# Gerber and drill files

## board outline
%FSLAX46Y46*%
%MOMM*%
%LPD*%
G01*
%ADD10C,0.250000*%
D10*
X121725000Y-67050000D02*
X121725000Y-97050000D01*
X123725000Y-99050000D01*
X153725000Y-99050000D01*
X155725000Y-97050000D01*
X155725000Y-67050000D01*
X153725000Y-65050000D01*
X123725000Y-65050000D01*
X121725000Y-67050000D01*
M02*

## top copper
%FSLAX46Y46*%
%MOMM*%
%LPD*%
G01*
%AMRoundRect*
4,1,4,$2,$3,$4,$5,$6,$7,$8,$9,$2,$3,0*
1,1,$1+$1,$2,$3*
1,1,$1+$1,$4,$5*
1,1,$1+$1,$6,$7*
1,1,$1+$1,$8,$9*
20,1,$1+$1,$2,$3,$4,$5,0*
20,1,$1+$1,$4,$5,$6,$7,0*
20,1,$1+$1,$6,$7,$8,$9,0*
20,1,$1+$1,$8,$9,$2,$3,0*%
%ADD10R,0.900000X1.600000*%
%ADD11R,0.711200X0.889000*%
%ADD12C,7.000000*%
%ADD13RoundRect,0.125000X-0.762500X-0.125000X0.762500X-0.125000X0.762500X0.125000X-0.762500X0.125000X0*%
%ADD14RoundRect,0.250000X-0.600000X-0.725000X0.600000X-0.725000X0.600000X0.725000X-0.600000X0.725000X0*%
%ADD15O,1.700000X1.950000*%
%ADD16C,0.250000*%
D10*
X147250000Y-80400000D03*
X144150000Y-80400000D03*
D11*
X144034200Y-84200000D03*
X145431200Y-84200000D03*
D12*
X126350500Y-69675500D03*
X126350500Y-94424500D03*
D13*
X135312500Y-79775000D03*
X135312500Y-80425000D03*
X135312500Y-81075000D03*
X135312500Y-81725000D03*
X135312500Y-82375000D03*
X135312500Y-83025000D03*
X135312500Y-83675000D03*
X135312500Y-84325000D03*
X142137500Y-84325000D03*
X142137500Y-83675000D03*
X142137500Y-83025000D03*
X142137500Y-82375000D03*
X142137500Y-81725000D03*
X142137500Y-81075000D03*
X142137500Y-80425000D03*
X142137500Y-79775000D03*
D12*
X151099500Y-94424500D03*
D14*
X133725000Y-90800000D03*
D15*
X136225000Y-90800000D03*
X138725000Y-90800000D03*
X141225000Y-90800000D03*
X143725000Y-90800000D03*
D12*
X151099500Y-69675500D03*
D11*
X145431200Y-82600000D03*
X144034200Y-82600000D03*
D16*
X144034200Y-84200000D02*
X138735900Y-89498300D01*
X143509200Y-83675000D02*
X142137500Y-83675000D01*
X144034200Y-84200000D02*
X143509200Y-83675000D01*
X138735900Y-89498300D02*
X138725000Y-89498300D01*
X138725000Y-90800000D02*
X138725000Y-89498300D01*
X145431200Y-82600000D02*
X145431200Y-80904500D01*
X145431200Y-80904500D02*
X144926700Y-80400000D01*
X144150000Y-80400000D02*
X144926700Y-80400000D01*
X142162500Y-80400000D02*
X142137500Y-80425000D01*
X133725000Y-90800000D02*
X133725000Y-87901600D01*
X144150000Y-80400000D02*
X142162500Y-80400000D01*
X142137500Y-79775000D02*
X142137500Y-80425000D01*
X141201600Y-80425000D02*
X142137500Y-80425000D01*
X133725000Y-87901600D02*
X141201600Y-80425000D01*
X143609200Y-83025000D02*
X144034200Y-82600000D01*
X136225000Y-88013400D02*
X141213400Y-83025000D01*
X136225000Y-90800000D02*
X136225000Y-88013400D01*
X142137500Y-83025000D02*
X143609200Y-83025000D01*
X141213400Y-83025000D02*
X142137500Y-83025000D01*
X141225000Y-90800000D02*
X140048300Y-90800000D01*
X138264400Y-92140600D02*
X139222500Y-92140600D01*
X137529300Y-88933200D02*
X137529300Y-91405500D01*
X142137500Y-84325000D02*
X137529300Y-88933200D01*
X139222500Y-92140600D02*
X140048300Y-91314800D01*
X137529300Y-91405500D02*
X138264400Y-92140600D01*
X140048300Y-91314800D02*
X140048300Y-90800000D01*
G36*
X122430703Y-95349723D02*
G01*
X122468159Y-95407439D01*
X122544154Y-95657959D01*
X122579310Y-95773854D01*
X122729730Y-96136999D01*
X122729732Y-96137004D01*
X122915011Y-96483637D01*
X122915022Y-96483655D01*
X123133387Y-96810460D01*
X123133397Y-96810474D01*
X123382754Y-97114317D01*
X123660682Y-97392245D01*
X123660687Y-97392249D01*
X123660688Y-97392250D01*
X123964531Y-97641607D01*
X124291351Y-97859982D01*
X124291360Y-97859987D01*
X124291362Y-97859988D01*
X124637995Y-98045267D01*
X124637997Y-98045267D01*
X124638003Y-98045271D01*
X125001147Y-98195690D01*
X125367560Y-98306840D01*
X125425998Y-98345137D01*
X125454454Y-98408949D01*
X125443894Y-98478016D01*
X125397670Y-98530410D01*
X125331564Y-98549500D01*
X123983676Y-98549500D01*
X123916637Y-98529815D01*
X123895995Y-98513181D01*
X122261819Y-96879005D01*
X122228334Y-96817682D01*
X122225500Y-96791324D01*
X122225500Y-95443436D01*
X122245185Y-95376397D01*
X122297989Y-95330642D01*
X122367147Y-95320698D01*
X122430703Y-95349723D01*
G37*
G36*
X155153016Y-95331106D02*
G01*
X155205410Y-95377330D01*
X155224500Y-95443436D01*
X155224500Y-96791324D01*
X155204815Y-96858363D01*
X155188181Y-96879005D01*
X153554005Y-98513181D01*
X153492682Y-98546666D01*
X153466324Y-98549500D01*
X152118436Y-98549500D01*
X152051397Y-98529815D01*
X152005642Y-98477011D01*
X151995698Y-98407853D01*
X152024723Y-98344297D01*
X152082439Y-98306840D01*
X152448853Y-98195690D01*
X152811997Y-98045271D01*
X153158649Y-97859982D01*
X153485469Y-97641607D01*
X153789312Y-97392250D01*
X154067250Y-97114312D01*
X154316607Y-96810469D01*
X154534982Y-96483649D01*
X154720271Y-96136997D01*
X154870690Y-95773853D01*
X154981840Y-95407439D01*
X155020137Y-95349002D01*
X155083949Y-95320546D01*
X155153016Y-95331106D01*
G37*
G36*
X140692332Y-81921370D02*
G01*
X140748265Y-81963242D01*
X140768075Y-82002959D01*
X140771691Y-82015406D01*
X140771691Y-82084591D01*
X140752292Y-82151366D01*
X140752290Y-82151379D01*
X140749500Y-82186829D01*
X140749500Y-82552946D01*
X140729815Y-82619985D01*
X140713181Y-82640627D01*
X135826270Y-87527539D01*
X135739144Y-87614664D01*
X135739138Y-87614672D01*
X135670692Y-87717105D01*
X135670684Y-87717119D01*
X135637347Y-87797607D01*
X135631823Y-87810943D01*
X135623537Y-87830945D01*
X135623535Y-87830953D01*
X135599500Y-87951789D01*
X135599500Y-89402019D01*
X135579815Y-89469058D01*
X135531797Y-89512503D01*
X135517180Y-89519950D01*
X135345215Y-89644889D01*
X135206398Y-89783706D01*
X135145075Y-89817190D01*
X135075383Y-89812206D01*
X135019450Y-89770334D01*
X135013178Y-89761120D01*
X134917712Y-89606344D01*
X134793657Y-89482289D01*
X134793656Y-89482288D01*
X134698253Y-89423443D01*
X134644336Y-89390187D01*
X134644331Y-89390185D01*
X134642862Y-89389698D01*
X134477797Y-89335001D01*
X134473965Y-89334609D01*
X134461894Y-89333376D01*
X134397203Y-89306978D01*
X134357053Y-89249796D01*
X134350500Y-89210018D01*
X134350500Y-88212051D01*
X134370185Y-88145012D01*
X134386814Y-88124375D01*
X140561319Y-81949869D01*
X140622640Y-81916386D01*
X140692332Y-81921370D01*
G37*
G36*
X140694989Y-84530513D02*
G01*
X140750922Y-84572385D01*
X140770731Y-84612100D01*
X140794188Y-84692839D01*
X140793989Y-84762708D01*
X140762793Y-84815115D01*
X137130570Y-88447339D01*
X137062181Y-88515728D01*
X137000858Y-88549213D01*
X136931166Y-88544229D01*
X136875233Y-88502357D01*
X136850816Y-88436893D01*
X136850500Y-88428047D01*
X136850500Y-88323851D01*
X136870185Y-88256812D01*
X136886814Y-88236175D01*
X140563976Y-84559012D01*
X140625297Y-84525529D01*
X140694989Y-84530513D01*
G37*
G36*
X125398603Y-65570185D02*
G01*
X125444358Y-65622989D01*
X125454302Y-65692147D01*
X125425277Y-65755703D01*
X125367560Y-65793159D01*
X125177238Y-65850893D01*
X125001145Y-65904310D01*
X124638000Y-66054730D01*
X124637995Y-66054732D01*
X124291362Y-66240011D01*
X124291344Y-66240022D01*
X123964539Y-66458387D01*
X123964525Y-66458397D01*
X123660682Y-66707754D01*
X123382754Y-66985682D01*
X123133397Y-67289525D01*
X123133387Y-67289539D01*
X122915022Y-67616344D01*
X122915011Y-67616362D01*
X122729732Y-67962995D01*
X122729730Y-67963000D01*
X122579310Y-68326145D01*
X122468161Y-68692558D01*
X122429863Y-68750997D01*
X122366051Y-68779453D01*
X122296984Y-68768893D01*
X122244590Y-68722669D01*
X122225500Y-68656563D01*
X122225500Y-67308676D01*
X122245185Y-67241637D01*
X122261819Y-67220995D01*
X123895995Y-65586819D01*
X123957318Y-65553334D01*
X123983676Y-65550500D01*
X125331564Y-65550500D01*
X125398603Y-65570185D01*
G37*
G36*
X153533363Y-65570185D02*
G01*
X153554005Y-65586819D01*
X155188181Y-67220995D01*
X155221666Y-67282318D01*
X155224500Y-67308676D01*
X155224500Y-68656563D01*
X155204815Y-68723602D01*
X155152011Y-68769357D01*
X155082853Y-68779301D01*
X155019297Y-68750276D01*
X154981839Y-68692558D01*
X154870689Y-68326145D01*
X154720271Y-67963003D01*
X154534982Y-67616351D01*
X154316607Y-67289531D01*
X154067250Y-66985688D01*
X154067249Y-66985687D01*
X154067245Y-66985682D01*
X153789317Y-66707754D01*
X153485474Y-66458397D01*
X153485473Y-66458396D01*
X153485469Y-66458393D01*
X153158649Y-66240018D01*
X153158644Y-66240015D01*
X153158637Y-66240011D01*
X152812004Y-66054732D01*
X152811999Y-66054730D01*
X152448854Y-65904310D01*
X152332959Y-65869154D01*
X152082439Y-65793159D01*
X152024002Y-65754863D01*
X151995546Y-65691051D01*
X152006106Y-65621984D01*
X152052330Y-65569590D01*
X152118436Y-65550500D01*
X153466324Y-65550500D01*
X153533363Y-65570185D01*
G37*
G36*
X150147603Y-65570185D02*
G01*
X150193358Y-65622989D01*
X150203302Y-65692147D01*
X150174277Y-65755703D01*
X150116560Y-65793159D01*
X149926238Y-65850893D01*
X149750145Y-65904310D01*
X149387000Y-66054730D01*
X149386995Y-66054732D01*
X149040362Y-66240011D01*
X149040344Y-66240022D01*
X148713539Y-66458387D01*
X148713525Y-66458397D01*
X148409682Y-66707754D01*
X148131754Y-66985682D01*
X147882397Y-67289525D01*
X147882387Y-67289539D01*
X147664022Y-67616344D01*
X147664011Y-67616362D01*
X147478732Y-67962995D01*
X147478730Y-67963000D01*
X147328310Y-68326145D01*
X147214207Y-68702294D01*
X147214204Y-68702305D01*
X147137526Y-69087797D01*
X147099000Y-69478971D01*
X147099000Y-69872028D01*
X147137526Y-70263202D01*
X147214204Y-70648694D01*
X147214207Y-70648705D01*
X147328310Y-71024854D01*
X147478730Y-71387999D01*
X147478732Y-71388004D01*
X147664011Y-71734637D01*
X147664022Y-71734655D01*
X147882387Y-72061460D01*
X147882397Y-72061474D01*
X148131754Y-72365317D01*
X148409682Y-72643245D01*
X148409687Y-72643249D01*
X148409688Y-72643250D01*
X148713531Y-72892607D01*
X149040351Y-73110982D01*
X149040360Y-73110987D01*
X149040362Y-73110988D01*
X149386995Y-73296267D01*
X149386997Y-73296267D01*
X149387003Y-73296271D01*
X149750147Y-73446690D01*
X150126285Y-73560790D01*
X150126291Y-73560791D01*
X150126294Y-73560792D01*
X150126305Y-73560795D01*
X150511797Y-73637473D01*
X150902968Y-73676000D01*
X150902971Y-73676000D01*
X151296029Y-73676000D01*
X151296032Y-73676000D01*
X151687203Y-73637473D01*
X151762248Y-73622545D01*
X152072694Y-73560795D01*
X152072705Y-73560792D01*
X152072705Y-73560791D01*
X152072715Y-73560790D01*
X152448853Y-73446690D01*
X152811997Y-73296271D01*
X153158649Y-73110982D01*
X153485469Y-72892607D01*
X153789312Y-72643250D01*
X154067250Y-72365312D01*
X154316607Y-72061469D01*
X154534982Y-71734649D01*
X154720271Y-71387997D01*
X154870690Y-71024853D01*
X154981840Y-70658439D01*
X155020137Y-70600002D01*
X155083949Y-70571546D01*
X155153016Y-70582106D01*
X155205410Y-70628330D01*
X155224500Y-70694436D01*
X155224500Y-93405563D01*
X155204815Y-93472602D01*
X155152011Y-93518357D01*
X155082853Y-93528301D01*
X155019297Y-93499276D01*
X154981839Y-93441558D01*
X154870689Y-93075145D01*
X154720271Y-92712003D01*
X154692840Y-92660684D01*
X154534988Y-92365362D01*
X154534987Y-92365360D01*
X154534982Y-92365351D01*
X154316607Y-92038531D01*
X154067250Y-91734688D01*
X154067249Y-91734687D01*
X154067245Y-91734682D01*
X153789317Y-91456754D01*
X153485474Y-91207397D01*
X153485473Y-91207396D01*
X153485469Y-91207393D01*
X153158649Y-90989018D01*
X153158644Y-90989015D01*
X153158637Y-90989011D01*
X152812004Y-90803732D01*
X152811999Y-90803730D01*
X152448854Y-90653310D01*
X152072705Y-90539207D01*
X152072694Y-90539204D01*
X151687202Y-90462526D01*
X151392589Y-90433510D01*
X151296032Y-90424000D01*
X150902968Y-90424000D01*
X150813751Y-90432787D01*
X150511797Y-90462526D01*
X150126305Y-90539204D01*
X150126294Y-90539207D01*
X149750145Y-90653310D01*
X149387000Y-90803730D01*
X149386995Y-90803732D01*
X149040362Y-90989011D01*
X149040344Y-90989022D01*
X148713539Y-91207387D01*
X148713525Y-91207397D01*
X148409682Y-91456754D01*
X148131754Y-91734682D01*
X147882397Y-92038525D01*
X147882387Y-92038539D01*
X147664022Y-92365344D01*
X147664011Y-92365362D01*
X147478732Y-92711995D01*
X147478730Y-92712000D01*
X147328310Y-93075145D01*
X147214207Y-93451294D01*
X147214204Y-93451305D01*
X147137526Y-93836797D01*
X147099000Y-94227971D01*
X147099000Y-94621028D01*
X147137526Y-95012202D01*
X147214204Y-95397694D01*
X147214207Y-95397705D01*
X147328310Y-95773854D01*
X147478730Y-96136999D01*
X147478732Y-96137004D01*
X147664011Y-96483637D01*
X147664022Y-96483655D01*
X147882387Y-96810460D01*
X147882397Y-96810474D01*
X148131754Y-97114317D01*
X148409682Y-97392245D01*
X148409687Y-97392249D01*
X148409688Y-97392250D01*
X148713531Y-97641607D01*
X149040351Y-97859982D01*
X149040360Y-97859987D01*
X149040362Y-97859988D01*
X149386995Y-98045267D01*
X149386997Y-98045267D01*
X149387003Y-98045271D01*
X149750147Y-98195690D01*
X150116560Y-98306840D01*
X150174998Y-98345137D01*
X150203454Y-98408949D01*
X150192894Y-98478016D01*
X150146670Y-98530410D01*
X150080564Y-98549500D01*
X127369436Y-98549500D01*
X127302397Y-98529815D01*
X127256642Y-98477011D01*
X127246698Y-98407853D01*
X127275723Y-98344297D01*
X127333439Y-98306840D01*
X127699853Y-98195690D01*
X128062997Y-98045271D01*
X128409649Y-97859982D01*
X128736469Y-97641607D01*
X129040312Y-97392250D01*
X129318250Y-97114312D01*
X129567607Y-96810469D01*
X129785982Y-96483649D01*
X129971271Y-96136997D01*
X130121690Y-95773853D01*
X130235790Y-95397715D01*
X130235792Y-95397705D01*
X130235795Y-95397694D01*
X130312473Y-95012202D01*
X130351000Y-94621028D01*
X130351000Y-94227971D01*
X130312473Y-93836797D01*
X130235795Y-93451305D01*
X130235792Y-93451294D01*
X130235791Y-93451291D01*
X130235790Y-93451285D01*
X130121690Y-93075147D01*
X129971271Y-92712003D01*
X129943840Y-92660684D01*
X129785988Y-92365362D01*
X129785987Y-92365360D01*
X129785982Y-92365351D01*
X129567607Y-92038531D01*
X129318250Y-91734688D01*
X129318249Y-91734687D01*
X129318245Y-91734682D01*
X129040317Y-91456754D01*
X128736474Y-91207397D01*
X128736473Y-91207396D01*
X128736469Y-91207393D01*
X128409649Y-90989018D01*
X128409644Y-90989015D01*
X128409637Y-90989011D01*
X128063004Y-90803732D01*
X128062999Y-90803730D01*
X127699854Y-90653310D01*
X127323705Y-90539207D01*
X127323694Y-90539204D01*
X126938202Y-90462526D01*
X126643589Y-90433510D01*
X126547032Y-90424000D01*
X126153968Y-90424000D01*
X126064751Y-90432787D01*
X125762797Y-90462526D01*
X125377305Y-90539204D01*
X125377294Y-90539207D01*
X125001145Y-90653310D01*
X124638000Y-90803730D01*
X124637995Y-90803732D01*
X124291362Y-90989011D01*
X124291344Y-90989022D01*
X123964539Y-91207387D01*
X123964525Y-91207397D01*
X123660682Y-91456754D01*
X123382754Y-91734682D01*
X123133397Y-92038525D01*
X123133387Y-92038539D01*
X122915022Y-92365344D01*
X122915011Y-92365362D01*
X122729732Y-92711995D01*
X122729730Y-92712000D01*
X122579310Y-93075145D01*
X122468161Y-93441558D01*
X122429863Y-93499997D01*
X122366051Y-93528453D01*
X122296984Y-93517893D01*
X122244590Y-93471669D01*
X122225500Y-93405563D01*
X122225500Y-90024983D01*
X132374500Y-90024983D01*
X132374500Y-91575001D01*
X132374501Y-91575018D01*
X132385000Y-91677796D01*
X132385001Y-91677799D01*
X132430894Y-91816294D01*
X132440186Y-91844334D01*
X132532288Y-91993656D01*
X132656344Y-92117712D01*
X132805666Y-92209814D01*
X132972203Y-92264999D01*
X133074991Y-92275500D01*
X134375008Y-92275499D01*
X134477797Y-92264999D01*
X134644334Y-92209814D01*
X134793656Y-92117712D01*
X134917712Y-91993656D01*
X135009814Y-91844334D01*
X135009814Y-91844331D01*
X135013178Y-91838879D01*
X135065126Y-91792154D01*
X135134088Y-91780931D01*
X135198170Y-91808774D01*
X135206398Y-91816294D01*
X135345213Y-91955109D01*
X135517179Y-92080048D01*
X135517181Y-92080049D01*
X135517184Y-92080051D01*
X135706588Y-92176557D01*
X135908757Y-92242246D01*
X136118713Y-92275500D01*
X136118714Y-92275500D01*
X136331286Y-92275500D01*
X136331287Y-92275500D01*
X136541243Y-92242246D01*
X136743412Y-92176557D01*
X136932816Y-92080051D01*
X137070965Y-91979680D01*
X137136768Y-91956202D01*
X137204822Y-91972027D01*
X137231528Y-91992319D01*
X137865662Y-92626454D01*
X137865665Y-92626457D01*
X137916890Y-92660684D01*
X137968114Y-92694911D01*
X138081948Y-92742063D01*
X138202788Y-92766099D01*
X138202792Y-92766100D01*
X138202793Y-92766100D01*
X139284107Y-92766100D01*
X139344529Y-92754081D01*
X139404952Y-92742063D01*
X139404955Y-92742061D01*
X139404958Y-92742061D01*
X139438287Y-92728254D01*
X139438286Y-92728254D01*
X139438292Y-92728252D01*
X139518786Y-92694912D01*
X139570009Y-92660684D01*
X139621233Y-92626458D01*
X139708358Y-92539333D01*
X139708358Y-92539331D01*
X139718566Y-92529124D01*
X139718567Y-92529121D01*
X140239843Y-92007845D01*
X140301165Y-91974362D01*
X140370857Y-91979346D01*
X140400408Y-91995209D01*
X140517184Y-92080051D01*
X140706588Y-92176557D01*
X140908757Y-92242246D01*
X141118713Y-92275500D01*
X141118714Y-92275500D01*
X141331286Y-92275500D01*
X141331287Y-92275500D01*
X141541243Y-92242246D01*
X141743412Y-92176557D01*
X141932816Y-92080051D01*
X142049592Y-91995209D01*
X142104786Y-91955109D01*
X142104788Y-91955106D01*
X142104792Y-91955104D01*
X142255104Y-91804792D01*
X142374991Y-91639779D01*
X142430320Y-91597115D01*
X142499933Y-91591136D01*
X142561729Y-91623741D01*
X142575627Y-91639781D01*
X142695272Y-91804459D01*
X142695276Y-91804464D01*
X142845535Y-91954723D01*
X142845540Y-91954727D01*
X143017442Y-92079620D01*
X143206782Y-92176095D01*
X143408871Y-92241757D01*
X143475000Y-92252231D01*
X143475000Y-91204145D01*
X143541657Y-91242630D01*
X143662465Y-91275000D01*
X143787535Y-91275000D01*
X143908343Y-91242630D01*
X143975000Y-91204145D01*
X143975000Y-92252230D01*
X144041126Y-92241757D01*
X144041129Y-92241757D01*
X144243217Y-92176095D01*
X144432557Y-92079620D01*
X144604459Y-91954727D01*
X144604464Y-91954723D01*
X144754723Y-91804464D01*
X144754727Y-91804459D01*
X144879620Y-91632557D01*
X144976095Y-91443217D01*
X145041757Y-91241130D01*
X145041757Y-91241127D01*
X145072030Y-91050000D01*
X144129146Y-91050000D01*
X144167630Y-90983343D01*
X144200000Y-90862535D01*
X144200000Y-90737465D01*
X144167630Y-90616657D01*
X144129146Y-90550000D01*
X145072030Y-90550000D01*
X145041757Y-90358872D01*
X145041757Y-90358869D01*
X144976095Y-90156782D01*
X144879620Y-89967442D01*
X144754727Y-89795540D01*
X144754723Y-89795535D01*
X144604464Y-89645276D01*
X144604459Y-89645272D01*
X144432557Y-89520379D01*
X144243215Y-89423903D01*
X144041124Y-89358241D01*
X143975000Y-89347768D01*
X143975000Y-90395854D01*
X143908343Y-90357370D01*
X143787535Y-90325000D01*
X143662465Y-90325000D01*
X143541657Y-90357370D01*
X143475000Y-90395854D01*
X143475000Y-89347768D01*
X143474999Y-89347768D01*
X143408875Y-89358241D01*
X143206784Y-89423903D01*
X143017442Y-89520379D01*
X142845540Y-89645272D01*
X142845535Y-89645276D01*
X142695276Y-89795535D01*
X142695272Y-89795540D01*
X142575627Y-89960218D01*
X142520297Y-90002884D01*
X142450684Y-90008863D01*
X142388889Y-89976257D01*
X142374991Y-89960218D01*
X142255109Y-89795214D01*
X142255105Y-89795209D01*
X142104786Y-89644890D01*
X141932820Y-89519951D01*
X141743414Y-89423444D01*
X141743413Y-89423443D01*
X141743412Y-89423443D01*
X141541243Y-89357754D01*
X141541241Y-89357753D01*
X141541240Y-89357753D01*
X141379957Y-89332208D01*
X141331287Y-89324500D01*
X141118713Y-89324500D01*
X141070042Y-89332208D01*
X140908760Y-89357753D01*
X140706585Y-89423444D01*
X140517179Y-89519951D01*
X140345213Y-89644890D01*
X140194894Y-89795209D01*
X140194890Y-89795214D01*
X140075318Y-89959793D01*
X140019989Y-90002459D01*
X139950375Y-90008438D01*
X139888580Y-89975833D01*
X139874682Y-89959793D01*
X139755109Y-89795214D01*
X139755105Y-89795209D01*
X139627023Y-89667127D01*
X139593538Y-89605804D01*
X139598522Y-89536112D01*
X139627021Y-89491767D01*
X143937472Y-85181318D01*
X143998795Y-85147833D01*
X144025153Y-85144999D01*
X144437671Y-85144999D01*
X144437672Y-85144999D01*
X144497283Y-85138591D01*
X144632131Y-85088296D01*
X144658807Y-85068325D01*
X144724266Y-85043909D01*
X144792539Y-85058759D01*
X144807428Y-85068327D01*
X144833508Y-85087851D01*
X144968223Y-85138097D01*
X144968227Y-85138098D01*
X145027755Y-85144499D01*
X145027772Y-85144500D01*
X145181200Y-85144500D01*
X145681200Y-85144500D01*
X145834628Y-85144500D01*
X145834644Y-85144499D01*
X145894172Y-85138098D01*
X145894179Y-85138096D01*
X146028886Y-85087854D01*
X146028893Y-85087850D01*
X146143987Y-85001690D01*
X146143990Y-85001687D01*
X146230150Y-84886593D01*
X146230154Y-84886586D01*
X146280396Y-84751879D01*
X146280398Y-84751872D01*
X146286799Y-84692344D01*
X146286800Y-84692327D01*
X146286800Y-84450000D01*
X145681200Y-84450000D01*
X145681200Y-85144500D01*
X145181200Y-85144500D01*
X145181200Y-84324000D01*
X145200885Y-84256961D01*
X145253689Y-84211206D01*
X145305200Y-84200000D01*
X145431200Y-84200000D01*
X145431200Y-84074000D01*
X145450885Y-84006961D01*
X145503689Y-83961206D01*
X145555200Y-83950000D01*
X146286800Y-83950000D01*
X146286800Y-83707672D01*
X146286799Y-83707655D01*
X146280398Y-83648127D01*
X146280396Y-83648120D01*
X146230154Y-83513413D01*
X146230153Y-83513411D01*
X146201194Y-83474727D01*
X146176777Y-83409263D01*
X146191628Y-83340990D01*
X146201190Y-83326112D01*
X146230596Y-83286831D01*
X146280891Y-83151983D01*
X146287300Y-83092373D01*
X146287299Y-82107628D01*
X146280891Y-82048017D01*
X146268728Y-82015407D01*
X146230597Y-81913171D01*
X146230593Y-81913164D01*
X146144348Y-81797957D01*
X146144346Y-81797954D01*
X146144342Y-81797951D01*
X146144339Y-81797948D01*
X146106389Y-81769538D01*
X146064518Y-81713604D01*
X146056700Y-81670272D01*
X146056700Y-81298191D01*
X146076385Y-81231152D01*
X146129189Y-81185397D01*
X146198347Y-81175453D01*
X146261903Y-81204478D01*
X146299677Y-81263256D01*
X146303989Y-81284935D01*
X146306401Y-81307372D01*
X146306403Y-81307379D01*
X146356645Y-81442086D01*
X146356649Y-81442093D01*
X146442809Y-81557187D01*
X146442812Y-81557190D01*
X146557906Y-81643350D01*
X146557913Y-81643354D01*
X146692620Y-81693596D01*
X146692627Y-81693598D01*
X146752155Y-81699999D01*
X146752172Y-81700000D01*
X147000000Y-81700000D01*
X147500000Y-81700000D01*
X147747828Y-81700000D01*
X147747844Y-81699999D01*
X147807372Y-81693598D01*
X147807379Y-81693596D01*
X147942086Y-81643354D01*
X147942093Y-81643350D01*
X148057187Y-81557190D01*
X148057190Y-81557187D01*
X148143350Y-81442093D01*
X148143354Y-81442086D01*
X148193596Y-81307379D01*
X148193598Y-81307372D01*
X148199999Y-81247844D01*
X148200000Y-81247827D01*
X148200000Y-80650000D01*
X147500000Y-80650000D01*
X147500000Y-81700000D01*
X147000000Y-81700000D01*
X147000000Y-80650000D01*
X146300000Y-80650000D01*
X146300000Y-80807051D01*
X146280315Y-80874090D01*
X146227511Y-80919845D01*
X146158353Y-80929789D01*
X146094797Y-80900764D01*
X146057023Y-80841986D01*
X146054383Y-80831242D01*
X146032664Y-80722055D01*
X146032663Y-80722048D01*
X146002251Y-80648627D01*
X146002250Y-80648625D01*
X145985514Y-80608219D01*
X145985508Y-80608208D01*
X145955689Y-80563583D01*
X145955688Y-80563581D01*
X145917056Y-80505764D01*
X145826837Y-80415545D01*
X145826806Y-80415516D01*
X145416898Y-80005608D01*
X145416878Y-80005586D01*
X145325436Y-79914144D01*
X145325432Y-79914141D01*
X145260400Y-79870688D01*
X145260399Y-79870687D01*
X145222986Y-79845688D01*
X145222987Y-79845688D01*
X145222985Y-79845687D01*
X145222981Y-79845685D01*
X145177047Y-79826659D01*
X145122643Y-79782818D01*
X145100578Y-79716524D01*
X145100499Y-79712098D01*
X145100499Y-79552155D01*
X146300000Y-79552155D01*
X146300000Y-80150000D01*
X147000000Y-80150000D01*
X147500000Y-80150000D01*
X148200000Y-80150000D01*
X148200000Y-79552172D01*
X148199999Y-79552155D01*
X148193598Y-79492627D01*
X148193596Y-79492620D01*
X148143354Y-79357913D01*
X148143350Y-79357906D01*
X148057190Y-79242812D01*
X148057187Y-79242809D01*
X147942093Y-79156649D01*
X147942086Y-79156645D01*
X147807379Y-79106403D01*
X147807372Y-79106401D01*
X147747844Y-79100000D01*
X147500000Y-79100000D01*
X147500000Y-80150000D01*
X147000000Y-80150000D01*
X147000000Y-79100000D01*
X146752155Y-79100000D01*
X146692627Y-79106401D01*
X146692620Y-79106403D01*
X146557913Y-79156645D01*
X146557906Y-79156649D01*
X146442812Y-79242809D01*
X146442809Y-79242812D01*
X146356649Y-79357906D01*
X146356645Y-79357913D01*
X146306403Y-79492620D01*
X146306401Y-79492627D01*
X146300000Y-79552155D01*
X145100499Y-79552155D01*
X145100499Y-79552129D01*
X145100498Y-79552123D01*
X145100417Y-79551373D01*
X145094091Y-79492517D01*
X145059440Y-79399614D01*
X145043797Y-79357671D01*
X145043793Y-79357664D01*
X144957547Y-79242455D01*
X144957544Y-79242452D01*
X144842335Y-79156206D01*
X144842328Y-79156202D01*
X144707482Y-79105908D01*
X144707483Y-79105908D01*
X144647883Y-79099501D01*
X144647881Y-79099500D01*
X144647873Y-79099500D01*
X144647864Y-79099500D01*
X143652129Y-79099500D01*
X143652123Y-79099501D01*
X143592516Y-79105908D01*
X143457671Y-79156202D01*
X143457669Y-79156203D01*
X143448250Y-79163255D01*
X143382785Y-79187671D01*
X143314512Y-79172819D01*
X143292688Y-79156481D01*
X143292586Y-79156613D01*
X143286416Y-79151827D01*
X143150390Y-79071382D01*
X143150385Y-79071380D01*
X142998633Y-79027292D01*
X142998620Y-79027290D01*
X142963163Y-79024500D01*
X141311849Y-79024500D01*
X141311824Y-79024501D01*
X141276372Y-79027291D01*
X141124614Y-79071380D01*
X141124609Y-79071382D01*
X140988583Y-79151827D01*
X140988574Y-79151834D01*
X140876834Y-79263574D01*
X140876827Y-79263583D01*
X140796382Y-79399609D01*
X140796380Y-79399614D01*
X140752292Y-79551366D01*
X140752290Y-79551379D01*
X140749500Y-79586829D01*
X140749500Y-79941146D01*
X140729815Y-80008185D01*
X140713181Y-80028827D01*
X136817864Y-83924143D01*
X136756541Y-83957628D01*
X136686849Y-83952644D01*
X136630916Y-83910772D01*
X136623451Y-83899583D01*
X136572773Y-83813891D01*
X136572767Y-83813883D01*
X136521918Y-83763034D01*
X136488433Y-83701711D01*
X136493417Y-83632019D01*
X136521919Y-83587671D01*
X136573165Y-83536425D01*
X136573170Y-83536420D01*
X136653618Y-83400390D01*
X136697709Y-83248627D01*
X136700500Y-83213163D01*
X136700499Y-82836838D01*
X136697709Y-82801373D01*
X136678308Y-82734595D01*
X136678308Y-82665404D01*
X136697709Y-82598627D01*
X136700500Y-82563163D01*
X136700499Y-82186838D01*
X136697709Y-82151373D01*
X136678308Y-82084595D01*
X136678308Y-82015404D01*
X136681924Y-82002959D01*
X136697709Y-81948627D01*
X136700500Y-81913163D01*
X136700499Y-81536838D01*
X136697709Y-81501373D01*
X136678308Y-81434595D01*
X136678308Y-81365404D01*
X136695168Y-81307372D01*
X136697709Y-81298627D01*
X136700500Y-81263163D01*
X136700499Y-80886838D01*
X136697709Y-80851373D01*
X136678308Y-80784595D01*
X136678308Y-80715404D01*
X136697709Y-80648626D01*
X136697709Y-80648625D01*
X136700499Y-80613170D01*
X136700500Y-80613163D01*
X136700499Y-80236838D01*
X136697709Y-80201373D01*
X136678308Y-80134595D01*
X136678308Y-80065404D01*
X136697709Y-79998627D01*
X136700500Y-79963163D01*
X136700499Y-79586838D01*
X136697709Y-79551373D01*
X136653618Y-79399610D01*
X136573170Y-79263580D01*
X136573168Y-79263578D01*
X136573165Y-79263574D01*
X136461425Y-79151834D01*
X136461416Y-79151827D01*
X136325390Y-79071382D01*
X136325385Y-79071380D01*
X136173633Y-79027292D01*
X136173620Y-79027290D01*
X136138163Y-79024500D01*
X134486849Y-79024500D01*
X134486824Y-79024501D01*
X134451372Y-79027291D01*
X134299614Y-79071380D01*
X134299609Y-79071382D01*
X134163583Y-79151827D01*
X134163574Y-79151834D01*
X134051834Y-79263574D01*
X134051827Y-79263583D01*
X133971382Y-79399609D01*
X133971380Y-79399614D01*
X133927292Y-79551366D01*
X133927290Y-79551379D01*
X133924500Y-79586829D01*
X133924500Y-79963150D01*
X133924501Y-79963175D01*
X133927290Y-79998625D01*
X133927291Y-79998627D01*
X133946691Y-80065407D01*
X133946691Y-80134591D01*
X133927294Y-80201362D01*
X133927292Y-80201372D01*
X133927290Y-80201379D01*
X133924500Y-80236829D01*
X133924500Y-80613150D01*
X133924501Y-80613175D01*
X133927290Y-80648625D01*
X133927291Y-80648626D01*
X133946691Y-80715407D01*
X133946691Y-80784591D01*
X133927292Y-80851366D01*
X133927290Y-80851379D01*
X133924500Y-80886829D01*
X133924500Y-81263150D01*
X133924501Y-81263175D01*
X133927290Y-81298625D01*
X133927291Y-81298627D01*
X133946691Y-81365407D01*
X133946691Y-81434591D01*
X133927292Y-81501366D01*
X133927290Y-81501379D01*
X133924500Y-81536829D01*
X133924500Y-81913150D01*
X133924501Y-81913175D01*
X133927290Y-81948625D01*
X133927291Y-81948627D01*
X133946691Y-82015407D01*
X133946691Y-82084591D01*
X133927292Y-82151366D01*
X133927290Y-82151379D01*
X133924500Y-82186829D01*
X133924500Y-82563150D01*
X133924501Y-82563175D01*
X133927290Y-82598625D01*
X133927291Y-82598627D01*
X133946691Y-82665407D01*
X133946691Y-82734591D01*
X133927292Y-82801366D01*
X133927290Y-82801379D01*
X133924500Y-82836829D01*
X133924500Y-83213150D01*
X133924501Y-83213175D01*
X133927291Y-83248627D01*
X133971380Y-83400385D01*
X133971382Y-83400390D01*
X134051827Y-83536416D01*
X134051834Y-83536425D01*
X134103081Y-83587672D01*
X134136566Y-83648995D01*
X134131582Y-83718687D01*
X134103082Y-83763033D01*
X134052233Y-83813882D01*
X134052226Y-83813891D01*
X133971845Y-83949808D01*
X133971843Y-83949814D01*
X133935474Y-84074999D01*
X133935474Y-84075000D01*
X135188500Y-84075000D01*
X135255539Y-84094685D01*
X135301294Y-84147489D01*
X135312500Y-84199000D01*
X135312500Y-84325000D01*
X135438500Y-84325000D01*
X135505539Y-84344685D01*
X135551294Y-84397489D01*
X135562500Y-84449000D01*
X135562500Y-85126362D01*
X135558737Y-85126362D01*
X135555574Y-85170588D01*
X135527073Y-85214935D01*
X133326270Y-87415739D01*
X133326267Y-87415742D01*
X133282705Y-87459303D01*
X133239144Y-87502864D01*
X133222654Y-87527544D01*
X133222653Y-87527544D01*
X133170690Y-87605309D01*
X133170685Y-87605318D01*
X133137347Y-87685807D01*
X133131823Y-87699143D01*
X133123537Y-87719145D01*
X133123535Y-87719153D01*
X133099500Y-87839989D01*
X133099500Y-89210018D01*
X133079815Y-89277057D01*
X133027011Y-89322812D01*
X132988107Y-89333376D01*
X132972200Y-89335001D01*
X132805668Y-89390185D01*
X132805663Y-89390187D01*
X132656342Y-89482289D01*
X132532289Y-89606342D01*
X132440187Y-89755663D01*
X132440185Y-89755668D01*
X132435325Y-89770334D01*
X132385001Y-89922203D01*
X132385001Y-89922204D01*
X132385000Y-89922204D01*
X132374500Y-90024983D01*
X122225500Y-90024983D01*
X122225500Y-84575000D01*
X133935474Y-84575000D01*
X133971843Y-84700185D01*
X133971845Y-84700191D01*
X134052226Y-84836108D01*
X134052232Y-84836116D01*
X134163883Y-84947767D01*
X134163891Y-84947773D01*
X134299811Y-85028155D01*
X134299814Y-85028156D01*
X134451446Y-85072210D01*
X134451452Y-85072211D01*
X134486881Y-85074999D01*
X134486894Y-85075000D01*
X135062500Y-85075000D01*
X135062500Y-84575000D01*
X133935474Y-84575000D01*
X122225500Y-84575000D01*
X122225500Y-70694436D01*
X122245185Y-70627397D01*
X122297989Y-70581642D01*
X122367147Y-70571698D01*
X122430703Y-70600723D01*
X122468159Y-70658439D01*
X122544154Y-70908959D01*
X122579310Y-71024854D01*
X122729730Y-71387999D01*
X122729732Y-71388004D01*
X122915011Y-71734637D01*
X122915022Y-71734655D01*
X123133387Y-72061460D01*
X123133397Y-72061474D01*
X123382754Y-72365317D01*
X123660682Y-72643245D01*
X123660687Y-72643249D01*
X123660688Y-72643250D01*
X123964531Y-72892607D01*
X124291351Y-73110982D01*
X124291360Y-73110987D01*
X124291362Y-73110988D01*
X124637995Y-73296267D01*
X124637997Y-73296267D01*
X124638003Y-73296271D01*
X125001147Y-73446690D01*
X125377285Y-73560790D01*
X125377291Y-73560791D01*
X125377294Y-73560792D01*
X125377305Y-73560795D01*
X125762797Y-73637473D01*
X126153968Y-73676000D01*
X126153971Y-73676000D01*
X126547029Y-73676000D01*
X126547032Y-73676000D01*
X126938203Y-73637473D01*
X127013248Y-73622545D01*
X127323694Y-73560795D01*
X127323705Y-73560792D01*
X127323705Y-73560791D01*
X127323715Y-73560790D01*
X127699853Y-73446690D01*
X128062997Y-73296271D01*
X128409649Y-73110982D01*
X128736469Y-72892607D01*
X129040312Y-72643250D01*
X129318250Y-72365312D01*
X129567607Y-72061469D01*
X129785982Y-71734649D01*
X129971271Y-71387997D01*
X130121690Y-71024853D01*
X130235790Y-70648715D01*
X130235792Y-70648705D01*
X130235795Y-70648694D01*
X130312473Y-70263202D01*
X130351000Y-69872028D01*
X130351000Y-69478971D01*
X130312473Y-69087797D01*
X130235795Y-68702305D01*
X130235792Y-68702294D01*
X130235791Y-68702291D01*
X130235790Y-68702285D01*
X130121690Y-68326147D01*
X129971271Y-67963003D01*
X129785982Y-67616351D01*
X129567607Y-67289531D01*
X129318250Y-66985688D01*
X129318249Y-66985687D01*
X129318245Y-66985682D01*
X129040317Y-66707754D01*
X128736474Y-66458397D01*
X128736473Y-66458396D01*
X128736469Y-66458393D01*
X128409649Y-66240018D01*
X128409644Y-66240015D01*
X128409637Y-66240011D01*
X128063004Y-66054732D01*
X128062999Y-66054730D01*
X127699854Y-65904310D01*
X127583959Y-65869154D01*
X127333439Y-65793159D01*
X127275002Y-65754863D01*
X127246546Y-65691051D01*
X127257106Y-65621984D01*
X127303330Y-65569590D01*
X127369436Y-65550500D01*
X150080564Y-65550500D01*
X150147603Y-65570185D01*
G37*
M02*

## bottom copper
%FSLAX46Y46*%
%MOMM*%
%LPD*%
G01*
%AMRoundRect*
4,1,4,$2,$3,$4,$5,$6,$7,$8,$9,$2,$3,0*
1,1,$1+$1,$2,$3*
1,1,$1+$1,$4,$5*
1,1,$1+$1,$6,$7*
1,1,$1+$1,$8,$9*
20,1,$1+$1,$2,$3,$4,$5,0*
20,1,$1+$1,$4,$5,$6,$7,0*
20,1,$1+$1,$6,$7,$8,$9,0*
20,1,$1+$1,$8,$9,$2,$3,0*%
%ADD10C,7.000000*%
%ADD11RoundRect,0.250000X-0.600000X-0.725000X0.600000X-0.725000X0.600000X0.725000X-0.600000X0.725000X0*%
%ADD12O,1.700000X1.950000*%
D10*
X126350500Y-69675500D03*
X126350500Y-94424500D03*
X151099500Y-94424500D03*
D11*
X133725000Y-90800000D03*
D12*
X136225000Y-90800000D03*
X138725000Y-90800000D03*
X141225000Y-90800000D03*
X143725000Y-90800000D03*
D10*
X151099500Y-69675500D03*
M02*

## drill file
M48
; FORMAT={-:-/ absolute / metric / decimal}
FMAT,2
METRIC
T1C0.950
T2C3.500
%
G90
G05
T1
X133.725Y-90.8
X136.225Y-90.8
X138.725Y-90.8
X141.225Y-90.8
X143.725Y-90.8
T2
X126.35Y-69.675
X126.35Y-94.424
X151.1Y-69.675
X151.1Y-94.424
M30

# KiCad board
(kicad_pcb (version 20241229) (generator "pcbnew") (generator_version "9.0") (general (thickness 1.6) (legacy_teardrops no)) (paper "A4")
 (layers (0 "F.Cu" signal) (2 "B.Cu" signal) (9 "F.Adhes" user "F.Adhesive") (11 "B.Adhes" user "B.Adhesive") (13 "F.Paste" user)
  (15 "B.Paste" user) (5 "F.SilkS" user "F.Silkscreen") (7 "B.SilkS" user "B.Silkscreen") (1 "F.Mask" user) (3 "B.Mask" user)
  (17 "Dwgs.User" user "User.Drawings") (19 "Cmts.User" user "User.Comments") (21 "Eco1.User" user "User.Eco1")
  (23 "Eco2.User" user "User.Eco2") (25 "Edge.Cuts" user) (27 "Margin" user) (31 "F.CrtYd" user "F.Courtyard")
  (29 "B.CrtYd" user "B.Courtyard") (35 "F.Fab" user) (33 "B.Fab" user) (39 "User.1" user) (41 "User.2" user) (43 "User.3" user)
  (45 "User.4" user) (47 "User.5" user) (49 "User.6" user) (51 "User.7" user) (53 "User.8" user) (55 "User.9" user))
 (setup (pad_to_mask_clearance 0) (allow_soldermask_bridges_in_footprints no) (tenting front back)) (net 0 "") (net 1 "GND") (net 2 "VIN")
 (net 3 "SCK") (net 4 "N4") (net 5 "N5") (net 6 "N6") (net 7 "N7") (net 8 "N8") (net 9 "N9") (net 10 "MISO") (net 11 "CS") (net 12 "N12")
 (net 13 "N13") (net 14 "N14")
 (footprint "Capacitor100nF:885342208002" (layer "F.Cu") (at 145.7 80.4 180)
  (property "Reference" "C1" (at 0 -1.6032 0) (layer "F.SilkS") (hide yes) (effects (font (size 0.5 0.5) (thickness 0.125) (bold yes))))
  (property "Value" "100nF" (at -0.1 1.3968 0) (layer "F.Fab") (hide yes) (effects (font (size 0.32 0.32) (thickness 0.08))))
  (pad "1" smd rect (at -1.55 0 180) (size 0.9 1.6) (layers "F.Cu" "F.Mask" "F.Paste") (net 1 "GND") (solder_mask_margin 0.102))
  (pad "2" smd rect (at 1.55 0 180) (size 0.9 1.6) (layers "F.Cu" "F.Mask" "F.Paste") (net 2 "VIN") (solder_mask_margin 0.102)))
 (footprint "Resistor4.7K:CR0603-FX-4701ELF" (layer "F.Cu") (at 144.7327 84.2)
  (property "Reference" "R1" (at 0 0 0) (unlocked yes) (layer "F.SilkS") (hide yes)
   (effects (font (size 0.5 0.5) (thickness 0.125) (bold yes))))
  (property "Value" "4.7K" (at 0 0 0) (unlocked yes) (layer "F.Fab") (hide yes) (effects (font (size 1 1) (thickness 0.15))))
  (pad "1" smd rect (at -0.6985 0) (size 0.7112 0.889) (layers "F.Cu" "F.Mask" "F.Paste") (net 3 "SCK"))
  (pad "2" smd rect (at 0.6985 0) (size 0.7112 0.889) (layers "F.Cu" "F.Mask" "F.Paste") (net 1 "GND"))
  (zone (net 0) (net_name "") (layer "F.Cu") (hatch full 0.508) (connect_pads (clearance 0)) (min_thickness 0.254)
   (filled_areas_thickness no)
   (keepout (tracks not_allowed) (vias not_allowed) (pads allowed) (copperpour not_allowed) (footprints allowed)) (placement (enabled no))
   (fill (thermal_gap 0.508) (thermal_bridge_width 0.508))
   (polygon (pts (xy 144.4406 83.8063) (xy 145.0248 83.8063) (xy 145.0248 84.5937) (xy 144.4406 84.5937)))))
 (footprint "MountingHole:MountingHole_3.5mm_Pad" (layer "F.Cu") (at 126.3505 69.6755)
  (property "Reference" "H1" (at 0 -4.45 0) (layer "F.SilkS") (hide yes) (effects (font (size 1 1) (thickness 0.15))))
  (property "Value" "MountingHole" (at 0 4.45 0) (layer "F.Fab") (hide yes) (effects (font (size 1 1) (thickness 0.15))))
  (pad "1" thru_hole circle (at 0 0) (size 7 7) (drill 3.5) (layers "*.Cu" "*.Mask") (remove_unused_layers no) (zone_connect 2)))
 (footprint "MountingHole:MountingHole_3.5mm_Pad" (layer "F.Cu") (at 126.3505 94.4245)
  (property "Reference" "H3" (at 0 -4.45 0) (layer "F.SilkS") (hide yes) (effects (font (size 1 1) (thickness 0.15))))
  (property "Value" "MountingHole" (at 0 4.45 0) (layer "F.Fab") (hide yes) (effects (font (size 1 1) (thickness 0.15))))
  (pad "1" thru_hole circle (at 0 0) (size 7 7) (drill 3.5) (layers "*.Cu" "*.Mask") (remove_unused_layers no) (zone_connect 2)))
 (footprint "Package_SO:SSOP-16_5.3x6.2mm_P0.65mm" (layer "F.Cu") (at 138.725 82.05)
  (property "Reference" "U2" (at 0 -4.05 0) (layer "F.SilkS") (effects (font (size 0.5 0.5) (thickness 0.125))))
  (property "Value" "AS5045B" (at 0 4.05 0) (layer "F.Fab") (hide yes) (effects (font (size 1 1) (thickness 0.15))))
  (pad "1" smd roundrect (at -3.4125 -2.275) (size 1.775 0.5) (layers "F.Cu" "F.Mask" "F.Paste") (roundrect_rratio 0.25) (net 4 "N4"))
  (pad "2" smd roundrect (at -3.4125 -1.625) (size 1.775 0.5) (layers "F.Cu" "F.Mask" "F.Paste") (roundrect_rratio 0.25) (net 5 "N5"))
  (pad "3" smd roundrect (at -3.4125 -0.975) (size 1.775 0.5) (layers "F.Cu" "F.Mask" "F.Paste") (roundrect_rratio 0.25) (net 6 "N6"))
  (pad "4" smd roundrect (at -3.4125 -0.325) (size 1.775 0.5) (layers "F.Cu" "F.Mask" "F.Paste") (roundrect_rratio 0.25) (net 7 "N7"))
  (pad "5" smd roundrect (at -3.4125 0.325) (size 1.775 0.5) (layers "F.Cu" "F.Mask" "F.Paste") (roundrect_rratio 0.25) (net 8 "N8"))
  (pad "6" smd roundrect (at -3.4125 0.975) (size 1.775 0.5) (layers "F.Cu" "F.Mask" "F.Paste") (roundrect_rratio 0.25) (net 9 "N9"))
  (pad "7" smd roundrect (at -3.4125 1.625) (size 1.775 0.5) (layers "F.Cu" "F.Mask" "F.Paste") (roundrect_rratio 0.25) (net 1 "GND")
   (zone_connect 2))
  (pad "8" smd roundrect (at -3.4125 2.275) (size 1.775 0.5) (layers "F.Cu" "F.Mask" "F.Paste") (roundrect_rratio 0.25) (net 1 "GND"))
  (pad "9" smd roundrect (at 3.4125 2.275) (size 1.775 0.5) (layers "F.Cu" "F.Mask" "F.Paste") (roundrect_rratio 0.25) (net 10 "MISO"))
  (pad "10" smd roundrect (at 3.4125 1.625) (size 1.775 0.5) (layers "F.Cu" "F.Mask" "F.Paste") (roundrect_rratio 0.25) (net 3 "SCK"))
  (pad "11" smd roundrect (at 3.4125 0.975) (size 1.775 0.5) (layers "F.Cu" "F.Mask" "F.Paste") (roundrect_rratio 0.25) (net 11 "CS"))
  (pad "12" smd roundrect (at 3.4125 0.325) (size 1.775 0.5) (layers "F.Cu" "F.Mask" "F.Paste") (roundrect_rratio 0.25) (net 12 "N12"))
  (pad "13" smd roundrect (at 3.4125 -0.325) (size 1.775 0.5) (layers "F.Cu" "F.Mask" "F.Paste") (roundrect_rratio 0.25) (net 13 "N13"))
  (pad "14" smd roundrect (at 3.4125 -0.975) (size 1.775 0.5) (layers "F.Cu" "F.Mask" "F.Paste") (roundrect_rratio 0.25) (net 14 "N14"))
  (pad "15" smd roundrect (at 3.4125 -1.625) (size 1.775 0.5) (layers "F.Cu" "F.Mask" "F.Paste") (roundrect_rratio 0.25) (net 2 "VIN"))
  (pad "16" smd roundrect (at 3.4125 -2.275) (size 1.775 0.5) (layers "F.Cu" "F.Mask" "F.Paste") (roundrect_rratio 0.25) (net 2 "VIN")))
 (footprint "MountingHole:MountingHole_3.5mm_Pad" (layer "F.Cu") (at 151.0995 94.4245)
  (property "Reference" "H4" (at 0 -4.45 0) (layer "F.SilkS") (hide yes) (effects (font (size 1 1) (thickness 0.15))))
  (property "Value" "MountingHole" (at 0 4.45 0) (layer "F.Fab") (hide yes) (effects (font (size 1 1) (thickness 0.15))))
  (pad "1" thru_hole circle (at 0 0) (size 7 7) (drill 3.5) (layers "*.Cu" "*.Mask") (remove_unused_layers no) (zone_connect 2)))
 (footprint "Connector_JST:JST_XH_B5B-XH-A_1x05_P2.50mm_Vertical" (layer "F.Cu") (at 133.725 90.8)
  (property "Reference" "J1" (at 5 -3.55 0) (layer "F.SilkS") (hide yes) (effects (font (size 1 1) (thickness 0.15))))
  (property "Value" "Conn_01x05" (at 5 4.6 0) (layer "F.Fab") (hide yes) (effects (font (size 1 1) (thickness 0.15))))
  (pad "1" thru_hole roundrect (at 0 0) (size 1.7 1.95) (drill 0.95) (layers "*.Cu" "*.Mask") (remove_unused_layers no)
   (roundrect_rratio 0.147059) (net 2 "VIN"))
  (pad "2" thru_hole oval (at 2.5 0) (size 1.7 1.95) (drill 0.95) (layers "*.Cu" "*.Mask") (remove_unused_layers no) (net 11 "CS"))
  (pad "3" thru_hole oval (at 5 0) (size 1.7 1.95) (drill 0.95) (layers "*.Cu" "*.Mask") (remove_unused_layers no) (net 3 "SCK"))
  (pad "4" thru_hole oval (at 7.5 0) (size 1.7 1.95) (drill 0.95) (layers "*.Cu" "*.Mask") (remove_unused_layers no) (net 10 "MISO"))
  (pad "5" thru_hole oval (at 10 0) (size 1.7 1.95) (drill 0.95) (layers "*.Cu" "*.Mask") (remove_unused_layers no) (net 1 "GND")))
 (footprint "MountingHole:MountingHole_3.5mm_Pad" (layer "F.Cu") (at 151.0995 69.6755)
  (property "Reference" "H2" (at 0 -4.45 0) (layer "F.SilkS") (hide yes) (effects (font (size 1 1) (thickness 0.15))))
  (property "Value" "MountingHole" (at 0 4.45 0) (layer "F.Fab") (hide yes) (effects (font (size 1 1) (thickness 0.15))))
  (pad "1" thru_hole circle (at 0 0) (size 7 7) (drill 3.5) (layers "*.Cu" "*.Mask") (remove_unused_layers no) (zone_connect 2)))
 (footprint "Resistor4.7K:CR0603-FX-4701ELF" (layer "F.Cu") (at 144.7327 82.6 180)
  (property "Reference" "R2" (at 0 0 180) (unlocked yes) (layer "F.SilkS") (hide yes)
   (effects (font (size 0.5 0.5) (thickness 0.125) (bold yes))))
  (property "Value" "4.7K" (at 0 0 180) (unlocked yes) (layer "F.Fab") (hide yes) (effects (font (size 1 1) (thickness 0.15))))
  (pad "1" smd rect (at -0.6985 0 180) (size 0.7112 0.889) (layers "F.Cu" "F.Mask" "F.Paste") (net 2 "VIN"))
  (pad "2" smd rect (at 0.6985 0 180) (size 0.7112 0.889) (layers "F.Cu" "F.Mask" "F.Paste") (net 11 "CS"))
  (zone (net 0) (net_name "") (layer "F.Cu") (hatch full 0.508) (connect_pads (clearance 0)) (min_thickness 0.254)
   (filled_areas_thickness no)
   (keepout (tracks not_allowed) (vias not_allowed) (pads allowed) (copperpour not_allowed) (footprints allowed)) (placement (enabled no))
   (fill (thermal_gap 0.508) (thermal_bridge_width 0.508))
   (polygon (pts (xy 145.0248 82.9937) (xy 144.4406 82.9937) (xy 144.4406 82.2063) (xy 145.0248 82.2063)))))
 (gr_poly
  (pts (xy 121.725 67.05) (xy 121.725 97.05) (xy 123.725 99.05) (xy 153.725 99.05) (xy 155.725 97.05) (xy 155.725 67.05) (xy 153.725 65.05)
   (xy 123.725 65.05))
  (stroke (width 0.25) (type solid)) (fill no) (layer "Edge.Cuts"))
 (segment (start 144.0342 84.2) (end 138.7359 89.4983) (width 0.25) (layer "F.Cu") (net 3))
 (segment (start 143.5092 83.675) (end 142.1375 83.675) (width 0.25) (layer "F.Cu") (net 3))
 (segment (start 144.0342 84.2) (end 143.5092 83.675) (width 0.25) (layer "F.Cu") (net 3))
 (segment (start 138.7359 89.4983) (end 138.725 89.4983) (width 0.25) (layer "F.Cu") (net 3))
 (segment (start 138.725 90.8) (end 138.725 89.4983) (width 0.25) (layer "F.Cu") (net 3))
 (segment (start 145.4312 82.6) (end 145.4312 80.9045) (width 0.25) (layer "F.Cu") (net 2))
 (segment (start 145.4312 80.9045) (end 144.9267 80.4) (width 0.25) (layer "F.Cu") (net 2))
 (segment (start 144.15 80.4) (end 144.9267 80.4) (width 0.25) (layer "F.Cu") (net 2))
 (segment (start 142.1625 80.4) (end 142.1375 80.425) (width 0.25) (layer "F.Cu") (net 2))
 (segment (start 133.725 90.8) (end 133.725 87.9016) (width 0.25) (layer "F.Cu") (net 2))
 (segment (start 144.15 80.4) (end 142.1625 80.4) (width 0.25) (layer "F.Cu") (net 2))
 (segment (start 142.1375 79.775) (end 142.1375 80.425) (width 0.25) (layer "F.Cu") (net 2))
 (segment (start 141.2016 80.425) (end 142.1375 80.425) (width 0.25) (layer "F.Cu") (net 2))
 (segment (start 133.725 87.9016) (end 141.2016 80.425) (width 0.25) (layer "F.Cu") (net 2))
 (segment (start 143.6092 83.025) (end 144.0342 82.6) (width 0.25) (layer "F.Cu") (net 11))
 (segment (start 136.225 88.0134) (end 141.2134 83.025) (width 0.25) (layer "F.Cu") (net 11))
 (segment (start 136.225 90.8) (end 136.225 88.0134) (width 0.25) (layer "F.Cu") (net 11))
 (segment (start 142.1375 83.025) (end 143.6092 83.025) (width 0.25) (layer "F.Cu") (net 11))
 (segment (start 141.2134 83.025) (end 142.1375 83.025) (width 0.25) (layer "F.Cu") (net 11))
 (segment (start 141.225 90.8) (end 140.0483 90.8) (width 0.25) (layer "F.Cu") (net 10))
 (segment (start 138.2644 92.1406) (end 139.2225 92.1406) (width 0.25) (layer "F.Cu") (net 10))
 (segment (start 137.5293 88.9332) (end 137.5293 91.4055) (width 0.25) (layer "F.Cu") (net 10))
 (segment (start 142.1375 84.325) (end 137.5293 88.9332) (width 0.25) (layer "F.Cu") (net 10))
 (segment (start 139.2225 92.1406) (end 140.0483 91.3148) (width 0.25) (layer "F.Cu") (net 10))
 (segment (start 137.5293 91.4055) (end 138.2644 92.1406) (width 0.25) (layer "F.Cu") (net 10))
 (segment (start 140.0483 91.3148) (end 140.0483 90.8) (width 0.25) (layer "F.Cu") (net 10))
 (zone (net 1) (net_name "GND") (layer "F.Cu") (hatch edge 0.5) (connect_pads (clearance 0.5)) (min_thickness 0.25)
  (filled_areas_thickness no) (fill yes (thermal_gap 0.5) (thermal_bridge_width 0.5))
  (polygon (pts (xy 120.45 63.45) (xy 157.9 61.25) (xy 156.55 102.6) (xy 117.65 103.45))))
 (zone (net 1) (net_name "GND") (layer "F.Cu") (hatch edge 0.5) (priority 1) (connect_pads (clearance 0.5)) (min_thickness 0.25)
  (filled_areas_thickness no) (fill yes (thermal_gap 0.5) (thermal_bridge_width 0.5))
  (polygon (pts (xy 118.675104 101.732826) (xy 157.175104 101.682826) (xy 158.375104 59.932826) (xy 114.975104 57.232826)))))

